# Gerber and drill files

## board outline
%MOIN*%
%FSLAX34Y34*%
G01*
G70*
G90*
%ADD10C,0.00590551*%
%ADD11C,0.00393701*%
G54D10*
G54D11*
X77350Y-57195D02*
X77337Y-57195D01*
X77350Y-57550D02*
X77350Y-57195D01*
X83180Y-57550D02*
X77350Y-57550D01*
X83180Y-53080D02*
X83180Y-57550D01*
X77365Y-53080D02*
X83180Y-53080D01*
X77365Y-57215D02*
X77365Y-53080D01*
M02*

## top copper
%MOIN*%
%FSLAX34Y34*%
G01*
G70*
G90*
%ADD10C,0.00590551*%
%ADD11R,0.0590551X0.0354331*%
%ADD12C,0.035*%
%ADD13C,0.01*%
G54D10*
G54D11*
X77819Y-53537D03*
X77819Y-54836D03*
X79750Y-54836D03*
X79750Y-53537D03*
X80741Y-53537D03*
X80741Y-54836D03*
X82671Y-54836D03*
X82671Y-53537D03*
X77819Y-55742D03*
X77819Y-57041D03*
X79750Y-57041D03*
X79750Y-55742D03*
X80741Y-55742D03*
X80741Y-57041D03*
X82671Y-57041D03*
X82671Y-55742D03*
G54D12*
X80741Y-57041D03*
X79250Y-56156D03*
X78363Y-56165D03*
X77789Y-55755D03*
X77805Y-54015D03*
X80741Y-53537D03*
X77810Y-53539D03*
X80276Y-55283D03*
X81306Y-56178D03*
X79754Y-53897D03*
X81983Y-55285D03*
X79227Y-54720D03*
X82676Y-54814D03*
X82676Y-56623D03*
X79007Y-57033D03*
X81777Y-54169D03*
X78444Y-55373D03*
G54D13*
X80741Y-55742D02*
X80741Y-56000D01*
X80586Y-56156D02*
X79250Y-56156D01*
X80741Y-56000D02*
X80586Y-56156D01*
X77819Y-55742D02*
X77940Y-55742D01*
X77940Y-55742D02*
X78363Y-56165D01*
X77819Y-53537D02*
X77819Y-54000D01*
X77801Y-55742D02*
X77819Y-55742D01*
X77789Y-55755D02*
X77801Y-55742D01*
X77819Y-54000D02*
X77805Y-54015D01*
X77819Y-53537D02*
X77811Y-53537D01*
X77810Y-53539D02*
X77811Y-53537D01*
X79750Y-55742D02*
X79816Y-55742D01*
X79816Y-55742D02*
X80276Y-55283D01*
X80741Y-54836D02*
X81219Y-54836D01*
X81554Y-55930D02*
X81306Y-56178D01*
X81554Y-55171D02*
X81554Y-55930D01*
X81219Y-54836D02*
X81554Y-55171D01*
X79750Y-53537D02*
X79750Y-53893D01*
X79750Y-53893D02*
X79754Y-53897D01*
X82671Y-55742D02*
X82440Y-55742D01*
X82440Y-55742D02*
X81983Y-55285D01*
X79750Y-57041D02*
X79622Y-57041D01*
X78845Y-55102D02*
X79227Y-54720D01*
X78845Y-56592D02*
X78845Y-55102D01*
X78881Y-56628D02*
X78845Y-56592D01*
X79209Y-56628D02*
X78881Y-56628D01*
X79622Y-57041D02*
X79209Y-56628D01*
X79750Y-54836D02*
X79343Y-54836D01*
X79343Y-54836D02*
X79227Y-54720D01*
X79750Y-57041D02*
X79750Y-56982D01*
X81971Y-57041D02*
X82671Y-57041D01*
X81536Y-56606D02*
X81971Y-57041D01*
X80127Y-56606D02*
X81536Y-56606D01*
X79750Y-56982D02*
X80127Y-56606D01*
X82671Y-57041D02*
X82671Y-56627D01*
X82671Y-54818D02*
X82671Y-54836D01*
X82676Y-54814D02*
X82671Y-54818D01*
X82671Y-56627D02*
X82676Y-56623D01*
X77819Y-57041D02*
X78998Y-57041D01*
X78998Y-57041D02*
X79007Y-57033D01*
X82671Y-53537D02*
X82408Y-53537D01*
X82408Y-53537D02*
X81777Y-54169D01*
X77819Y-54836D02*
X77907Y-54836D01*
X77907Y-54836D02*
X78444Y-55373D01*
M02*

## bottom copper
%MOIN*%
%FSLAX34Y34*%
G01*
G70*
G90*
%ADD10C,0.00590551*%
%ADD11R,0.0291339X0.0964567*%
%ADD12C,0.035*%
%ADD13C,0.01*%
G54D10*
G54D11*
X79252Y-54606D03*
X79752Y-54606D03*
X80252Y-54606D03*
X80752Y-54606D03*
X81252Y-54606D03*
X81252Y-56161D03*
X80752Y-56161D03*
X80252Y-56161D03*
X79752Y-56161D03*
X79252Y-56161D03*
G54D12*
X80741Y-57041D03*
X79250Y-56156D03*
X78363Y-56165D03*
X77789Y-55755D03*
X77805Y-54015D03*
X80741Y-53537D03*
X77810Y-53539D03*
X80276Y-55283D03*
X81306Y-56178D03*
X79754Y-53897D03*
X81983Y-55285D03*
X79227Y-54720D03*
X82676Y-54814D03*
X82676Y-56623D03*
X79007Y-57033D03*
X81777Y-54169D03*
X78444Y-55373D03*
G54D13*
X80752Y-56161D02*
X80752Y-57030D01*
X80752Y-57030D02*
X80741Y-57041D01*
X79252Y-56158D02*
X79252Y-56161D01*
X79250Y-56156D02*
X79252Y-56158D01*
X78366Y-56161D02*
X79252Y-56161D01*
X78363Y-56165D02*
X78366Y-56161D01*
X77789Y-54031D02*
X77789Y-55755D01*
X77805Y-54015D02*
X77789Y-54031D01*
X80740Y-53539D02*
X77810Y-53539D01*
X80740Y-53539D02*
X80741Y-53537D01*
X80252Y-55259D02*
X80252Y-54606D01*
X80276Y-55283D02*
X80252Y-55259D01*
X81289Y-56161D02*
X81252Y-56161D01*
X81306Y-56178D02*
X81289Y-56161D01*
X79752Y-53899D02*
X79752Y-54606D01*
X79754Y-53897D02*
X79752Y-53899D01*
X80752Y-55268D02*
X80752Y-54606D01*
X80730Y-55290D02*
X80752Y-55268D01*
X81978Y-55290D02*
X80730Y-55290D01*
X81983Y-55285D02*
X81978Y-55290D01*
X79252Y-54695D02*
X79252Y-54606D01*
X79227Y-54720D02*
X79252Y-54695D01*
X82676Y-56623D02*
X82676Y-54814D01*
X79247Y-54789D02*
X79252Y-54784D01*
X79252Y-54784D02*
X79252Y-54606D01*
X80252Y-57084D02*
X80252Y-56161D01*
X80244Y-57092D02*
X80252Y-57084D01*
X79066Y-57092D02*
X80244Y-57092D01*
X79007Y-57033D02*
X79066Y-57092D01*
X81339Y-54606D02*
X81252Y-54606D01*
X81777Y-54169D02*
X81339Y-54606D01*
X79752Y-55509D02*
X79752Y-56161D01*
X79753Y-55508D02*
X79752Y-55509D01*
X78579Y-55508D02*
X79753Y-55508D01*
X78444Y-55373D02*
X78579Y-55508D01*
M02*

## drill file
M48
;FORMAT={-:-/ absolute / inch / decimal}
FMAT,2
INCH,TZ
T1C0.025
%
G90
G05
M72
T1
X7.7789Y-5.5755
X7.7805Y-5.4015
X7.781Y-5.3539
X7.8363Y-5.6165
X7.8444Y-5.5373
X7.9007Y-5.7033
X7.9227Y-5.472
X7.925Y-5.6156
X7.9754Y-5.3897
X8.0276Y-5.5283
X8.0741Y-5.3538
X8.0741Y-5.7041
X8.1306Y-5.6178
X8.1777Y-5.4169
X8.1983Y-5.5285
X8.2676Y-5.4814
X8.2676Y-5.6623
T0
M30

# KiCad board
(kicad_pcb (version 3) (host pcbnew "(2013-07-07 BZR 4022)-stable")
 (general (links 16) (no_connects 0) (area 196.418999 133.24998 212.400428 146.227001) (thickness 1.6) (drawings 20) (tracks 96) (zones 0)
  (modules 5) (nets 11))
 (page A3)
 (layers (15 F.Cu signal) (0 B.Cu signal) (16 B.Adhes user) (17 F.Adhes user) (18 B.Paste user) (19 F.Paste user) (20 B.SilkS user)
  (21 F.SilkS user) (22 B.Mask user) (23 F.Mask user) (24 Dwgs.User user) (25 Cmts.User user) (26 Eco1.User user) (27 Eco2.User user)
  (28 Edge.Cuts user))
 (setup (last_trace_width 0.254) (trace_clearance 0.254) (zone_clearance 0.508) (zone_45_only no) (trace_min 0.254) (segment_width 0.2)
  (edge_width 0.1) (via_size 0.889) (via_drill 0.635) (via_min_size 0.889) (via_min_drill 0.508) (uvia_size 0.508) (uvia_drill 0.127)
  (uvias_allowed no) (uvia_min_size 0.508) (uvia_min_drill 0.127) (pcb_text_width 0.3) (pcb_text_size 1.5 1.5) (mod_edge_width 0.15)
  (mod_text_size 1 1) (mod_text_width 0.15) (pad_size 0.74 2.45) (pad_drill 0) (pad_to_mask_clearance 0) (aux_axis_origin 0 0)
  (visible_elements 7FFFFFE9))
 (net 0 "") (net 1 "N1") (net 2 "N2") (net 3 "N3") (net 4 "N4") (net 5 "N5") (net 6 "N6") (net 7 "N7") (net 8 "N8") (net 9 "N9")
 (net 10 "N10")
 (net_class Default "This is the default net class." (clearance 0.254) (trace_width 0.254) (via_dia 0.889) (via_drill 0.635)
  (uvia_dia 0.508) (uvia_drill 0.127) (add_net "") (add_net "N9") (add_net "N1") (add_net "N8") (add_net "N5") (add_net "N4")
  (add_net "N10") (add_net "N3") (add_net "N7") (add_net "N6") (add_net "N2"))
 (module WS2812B (layer F.Cu) (at 200.1139 137.63498)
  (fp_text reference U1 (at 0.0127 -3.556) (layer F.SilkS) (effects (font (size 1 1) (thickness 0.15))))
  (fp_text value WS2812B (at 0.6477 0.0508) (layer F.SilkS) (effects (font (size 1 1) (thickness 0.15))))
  (pad 1 smd rect (at -2.45184 -1.64878) (size 1.5 0.9) (layers F.Cu F.Paste F.Mask) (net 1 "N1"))
  (pad 2 smd rect (at -2.45184 1.64878) (size 1.5 0.9) (layers F.Cu F.Paste F.Mask) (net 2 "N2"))
  (pad 3 smd rect (at 2.45184 1.64878) (size 1.5 0.9) (layers F.Cu F.Paste F.Mask) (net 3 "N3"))
  (pad 4 smd rect (at 2.45184 -1.64878) (size 1.5 0.9) (layers F.Cu F.Paste F.Mask) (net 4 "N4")))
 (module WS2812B (layer F.Cu) (at 207.53484 137.63498)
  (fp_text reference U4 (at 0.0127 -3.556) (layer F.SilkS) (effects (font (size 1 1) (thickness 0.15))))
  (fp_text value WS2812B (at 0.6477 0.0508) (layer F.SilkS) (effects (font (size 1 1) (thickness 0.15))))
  (pad 1 smd rect (at -2.45184 -1.64878) (size 1.5 0.9) (layers F.Cu F.Paste F.Mask) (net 1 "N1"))
  (pad 2 smd rect (at -2.45184 1.64878) (size 1.5 0.9) (layers F.Cu F.Paste F.Mask) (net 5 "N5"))
  (pad 3 smd rect (at 2.45184 1.64878) (size 1.5 0.9) (layers F.Cu F.Paste F.Mask) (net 3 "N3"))
  (pad 4 smd rect (at 2.45184 -1.64878) (size 1.5 0.9) (layers F.Cu F.Paste F.Mask) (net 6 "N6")))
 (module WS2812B (layer F.Cu) (at 200.1139 143.23568)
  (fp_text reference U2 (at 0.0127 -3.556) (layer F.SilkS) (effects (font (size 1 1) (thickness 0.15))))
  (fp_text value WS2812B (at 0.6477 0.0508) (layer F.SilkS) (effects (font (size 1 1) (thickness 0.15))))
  (pad 1 smd rect (at -2.45184 -1.64878) (size 1.5 0.9) (layers F.Cu F.Paste F.Mask) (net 1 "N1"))
  (pad 2 smd rect (at -2.45184 1.64878) (size 1.5 0.9) (layers F.Cu F.Paste F.Mask) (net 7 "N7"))
  (pad 3 smd rect (at 2.45184 1.64878) (size 1.5 0.9) (layers F.Cu F.Paste F.Mask) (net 3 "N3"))
  (pad 4 smd rect (at 2.45184 -1.64878) (size 1.5 0.9) (layers F.Cu F.Paste F.Mask) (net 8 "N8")))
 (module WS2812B (layer F.Cu) (at 207.53484 143.23568)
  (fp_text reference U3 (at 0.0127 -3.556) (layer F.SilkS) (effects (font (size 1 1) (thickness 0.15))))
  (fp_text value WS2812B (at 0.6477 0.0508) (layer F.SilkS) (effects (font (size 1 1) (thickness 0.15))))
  (pad 1 smd rect (at -2.45184 -1.64878) (size 1.5 0.9) (layers F.Cu F.Paste F.Mask) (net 1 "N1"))
  (pad 2 smd rect (at -2.45184 1.64878) (size 1.5 0.9) (layers F.Cu F.Paste F.Mask) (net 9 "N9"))
  (pad 3 smd rect (at 2.45184 1.64878) (size 1.5 0.9) (layers F.Cu F.Paste F.Mask) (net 3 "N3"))
  (pad 4 smd rect (at 2.45184 -1.64878) (size 1.5 0.9) (layers F.Cu F.Paste F.Mask) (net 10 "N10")))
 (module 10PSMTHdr (layer F.Cu) (at 207.01 139.7)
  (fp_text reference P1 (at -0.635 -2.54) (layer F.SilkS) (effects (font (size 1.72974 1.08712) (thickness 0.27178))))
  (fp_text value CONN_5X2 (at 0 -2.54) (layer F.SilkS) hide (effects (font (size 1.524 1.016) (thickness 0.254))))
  (pad 2 smd rect (at -5.70992 -1) (size 0.74 2.45) (layers B.Cu B.Paste B.Mask) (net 3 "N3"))
  (pad 4 smd rect (at -4.43992 -1) (size 0.74 2.45) (layers B.Cu B.Paste B.Mask) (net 4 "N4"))
  (pad 6 smd rect (at -3.16992 -1) (size 0.74 2.45) (layers B.Cu B.Paste B.Mask) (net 8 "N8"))
  (pad 8 smd rect (at -1.89992 -1) (size 0.74 2.45) (layers B.Cu B.Paste B.Mask) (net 10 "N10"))
  (pad 10 smd rect (at -0.62992 -1) (size 0.74 2.45) (layers B.Cu B.Paste B.Mask) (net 6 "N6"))
  (pad 9 smd rect (at -0.62992 2.95) (size 0.74 2.45) (layers B.Cu B.Paste B.Mask) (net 5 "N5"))
  (pad 7 smd rect (at -1.89992 2.95) (size 0.74 2.45) (layers B.Cu B.Paste B.Mask) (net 9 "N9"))
  (pad 5 smd rect (at -3.16992 2.95) (size 0.74 2.45) (layers B.Cu B.Paste B.Mask) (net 7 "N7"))
  (pad 3 smd rect (at -4.43992 2.95) (size 0.74 2.45) (layers B.Cu B.Paste B.Mask) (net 2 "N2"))
  (pad 1 smd rect (at -5.70992 2.95) (size 0.74 2.45) (layers B.Cu B.Paste B.Mask) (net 1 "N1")))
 (gr_line (start 196.469 145.2753) (end 196.43598 145.2753) (angle 90) (layer Edge.Cuts) (width 0.1))
 (gr_line (start 196.469 146.177) (end 196.469 145.2753) (angle 90) (layer Edge.Cuts) (width 0.1))
 (gr_line (start 211.2772 146.177) (end 196.469 146.177) (angle 90) (layer Edge.Cuts) (width 0.1))
 (gr_line (start 211.2772 134.8232) (end 211.2772 146.177) (angle 90) (layer Edge.Cuts) (width 0.1))
 (gr_line (start 196.5071 134.8232) (end 211.2772 134.8232) (angle 90) (layer Edge.Cuts) (width 0.1))
 (gr_line (start 196.5071 145.3261) (end 196.5071 134.8232) (angle 90) (layer Edge.Cuts) (width 0.1))
 (via (at 205.083 144.88446) (size 0.889) (layers F.Cu B.Cu) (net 9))
 (segment (start 205.11008 142.65) (end 205.11008 144.85738) (width 0.254) (layer B.Cu) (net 9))
 (segment (start 205.11008 144.85738) (end 205.083 144.88446) (width 0.254) (layer B.Cu) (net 9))
 (segment (start 205.083 141.5869) (end 205.083 142.24168) (width 0.254) (layer F.Cu) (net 1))
 (segment (start 201.30008 142.64132) (end 201.30008 142.65) (width 0.254) (layer B.Cu) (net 1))
 (segment (start 201.295 142.63624) (end 201.30008 142.64132) (width 0.254) (layer B.Cu) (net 1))
 (via (at 201.295 142.63624) (size 0.889) (layers F.Cu B.Cu) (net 1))
 (segment (start 204.68844 142.63624) (end 201.295 142.63624) (width 0.254) (layer F.Cu) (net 1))
 (segment (start 205.083 142.24168) (end 204.68844 142.63624) (width 0.254) (layer F.Cu) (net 1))
 (segment (start 197.66206 141.5869) (end 197.96982 141.5869) (width 0.254) (layer F.Cu) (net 1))
 (segment (start 199.05112 142.65) (end 201.30008 142.65) (width 0.254) (layer B.Cu) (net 1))
 (segment (start 199.04202 142.6591) (end 199.05112 142.65) (width 0.254) (layer B.Cu) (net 1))
 (via (at 199.04202 142.6591) (size 0.889) (layers F.Cu B.Cu) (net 1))
 (segment (start 197.96982 141.5869) (end 199.04202 142.6591) (width 0.254) (layer F.Cu) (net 1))
 (segment (start 197.66206 135.9862) (end 197.66206 137.16074) (width 0.254) (layer F.Cu) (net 1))
 (segment (start 197.61486 141.5869) (end 197.66206 141.5869) (width 0.254) (layer F.Cu) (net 1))
 (segment (start 197.58406 141.6177) (end 197.61486 141.5869) (width 0.254) (layer F.Cu) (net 1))
 (via (at 197.58406 141.6177) (size 0.889) (layers F.Cu B.Cu) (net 1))
 (segment (start 197.58406 137.23874) (end 197.58406 141.6177) (width 0.254) (layer B.Cu) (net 1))
 (segment (start 197.6247 137.1981) (end 197.58406 137.23874) (width 0.254) (layer B.Cu) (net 1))
 (via (at 197.6247 137.1981) (size 0.889) (layers F.Cu B.Cu) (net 1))
 (segment (start 197.66206 137.16074) (end 197.6247 137.1981) (width 0.254) (layer F.Cu) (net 1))
 (via (at 205.083 135.9862) (size 0.889) (layers F.Cu B.Cu) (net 1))
 (segment (start 197.66206 135.9862) (end 197.64026 135.9862) (width 0.254) (layer F.Cu) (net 1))
 (segment (start 197.6374 135.98906) (end 197.64026 135.9862) (width 0.254) (layer F.Cu) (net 1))
 (via (at 197.6374 135.98906) (size 0.889) (layers F.Cu B.Cu) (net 1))
 (segment (start 205.08014 135.98906) (end 197.6374 135.98906) (width 0.254) (layer B.Cu) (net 1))
 (segment (start 205.08014 135.98906) (end 205.083 135.9862) (width 0.254) (layer B.Cu) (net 1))
 (segment (start 202.56574 141.5869) (end 202.73296 141.5869) (width 0.254) (layer F.Cu) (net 8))
 (segment (start 203.84008 140.35786) (end 203.84008 138.7) (width 0.254) (layer B.Cu) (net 8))
 (segment (start 203.90104 140.41882) (end 203.84008 140.35786) (width 0.254) (layer B.Cu) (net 8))
 (via (at 203.90104 140.41882) (size 0.889) (layers F.Cu B.Cu) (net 8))
 (segment (start 202.73296 141.5869) (end 203.90104 140.41882) (width 0.254) (layer F.Cu) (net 8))
 (segment (start 205.083 139.28376) (end 206.29658 139.28376) (width 0.254) (layer F.Cu) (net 5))
 (segment (start 206.47512 142.65) (end 206.38008 142.65) (width 0.254) (layer B.Cu) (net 5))
 (segment (start 206.51724 142.69212) (end 206.47512 142.65) (width 0.254) (layer B.Cu) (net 5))
 (via (at 206.51724 142.69212) (size 0.889) (layers F.Cu B.Cu) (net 5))
 (segment (start 207.14716 142.0622) (end 206.51724 142.69212) (width 0.254) (layer F.Cu) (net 5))
 (segment (start 207.14716 140.13434) (end 207.14716 142.0622) (width 0.254) (layer F.Cu) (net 5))
 (segment (start 206.29658 139.28376) (end 207.14716 140.13434) (width 0.254) (layer F.Cu) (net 5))
 (segment (start 202.56574 135.9862) (end 202.56574 136.88896) (width 0.254) (layer F.Cu) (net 4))
 (segment (start 202.57008 136.90346) (end 202.57008 138.7) (width 0.254) (layer B.Cu) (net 4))
 (segment (start 202.57516 136.89838) (end 202.57008 136.90346) (width 0.254) (layer B.Cu) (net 4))
 (via (at 202.57516 136.89838) (size 0.889) (layers F.Cu B.Cu) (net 4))
 (segment (start 202.56574 136.88896) (end 202.57516 136.89838) (width 0.254) (layer F.Cu) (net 4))
 (segment (start 209.98668 141.5869) (end 209.39982 141.5869) (width 0.254) (layer F.Cu) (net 10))
 (segment (start 205.11008 140.38072) (end 205.11008 138.7) (width 0.254) (layer B.Cu) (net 10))
 (segment (start 205.0542 140.4366) (end 205.11008 140.38072) (width 0.254) (layer B.Cu) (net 10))
 (segment (start 208.22412 140.4366) (end 205.0542 140.4366) (width 0.254) (layer B.Cu) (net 10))
 (segment (start 208.23682 140.4239) (end 208.22412 140.4366) (width 0.254) (layer B.Cu) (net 10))
 (via (at 208.23682 140.4239) (size 0.889) (layers F.Cu B.Cu) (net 10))
 (segment (start 209.39982 141.5869) (end 208.23682 140.4239) (width 0.254) (layer F.Cu) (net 10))
 (segment (start 202.56574 144.88446) (end 202.2402 144.88446) (width 0.254) (layer F.Cu) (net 3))
 (segment (start 200.2663 139.95908) (end 201.23658 138.9888) (width 0.254) (layer F.Cu) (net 3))
 (segment (start 200.2663 143.74368) (end 200.2663 139.95908) (width 0.254) (layer F.Cu) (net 3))
 (segment (start 200.35774 143.83512) (end 200.2663 143.74368) (width 0.254) (layer F.Cu) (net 3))
 (segment (start 201.19086 143.83512) (end 200.35774 143.83512) (width 0.254) (layer F.Cu) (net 3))
 (segment (start 202.2402 144.88446) (end 201.19086 143.83512) (width 0.254) (layer F.Cu) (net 3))
 (segment (start 202.56574 139.28376) (end 201.53154 139.28376) (width 0.254) (layer F.Cu) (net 3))
 (segment (start 201.53154 139.28376) (end 201.23658 138.9888) (width 0.254) (layer F.Cu) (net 3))
 (segment (start 201.30008 138.9253) (end 201.30008 138.7) (width 0.254) (layer B.Cu) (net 3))
 (via (at 201.23658 138.9888) (size 0.889) (layers F.Cu B.Cu) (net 3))
 (segment (start 201.23658 138.9888) (end 201.30008 138.9253) (width 0.254) (layer B.Cu) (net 3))
 (segment (start 202.56574 144.88446) (end 202.56574 144.73608) (width 0.254) (layer F.Cu) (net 3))
 (segment (start 208.20666 144.88446) (end 209.98668 144.88446) (width 0.254) (layer F.Cu) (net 3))
 (segment (start 207.10144 143.77924) (end 208.20666 144.88446) (width 0.254) (layer F.Cu) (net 3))
 (segment (start 203.52258 143.77924) (end 207.10144 143.77924) (width 0.254) (layer F.Cu) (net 3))
 (segment (start 202.56574 144.73608) (end 203.52258 143.77924) (width 0.254) (layer F.Cu) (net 3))
 (segment (start 209.98668 144.88446) (end 209.98668 143.83278) (width 0.254) (layer F.Cu) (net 3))
 (segment (start 209.98668 139.23792) (end 209.98668 139.28376) (width 0.254) (layer F.Cu) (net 3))
 (segment (start 209.99704 139.22756) (end 209.98668 139.23792) (width 0.254) (layer F.Cu) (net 3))
 (via (at 209.99704 139.22756) (size 0.889) (layers F.Cu B.Cu) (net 3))
 (segment (start 209.99704 143.82242) (end 209.99704 139.22756) (width 0.254) (layer B.Cu) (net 3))
 (via (at 209.99704 143.82242) (size 0.889) (layers F.Cu B.Cu) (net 3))
 (segment (start 209.98668 143.83278) (end 209.99704 143.82242) (width 0.254) (layer F.Cu) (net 3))
 (segment (start 201.28738 139.16406) (end 201.30008 139.15136) (width 0.254) (layer B.Cu) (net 3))
 (segment (start 201.30008 139.15136) (end 201.30008 138.7) (width 0.254) (layer B.Cu) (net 3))
 (segment (start 197.66206 144.88446) (end 200.65714 144.88446) (width 0.254) (layer F.Cu) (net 7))
 (segment (start 203.84008 144.99336) (end 203.84008 142.65) (width 0.254) (layer B.Cu) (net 7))
 (segment (start 203.81976 145.01368) (end 203.84008 144.99336) (width 0.254) (layer B.Cu) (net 7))
 (segment (start 200.82764 145.01368) (end 203.81976 145.01368) (width 0.254) (layer B.Cu) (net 7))
 (segment (start 200.67778 144.86382) (end 200.82764 145.01368) (width 0.254) (layer B.Cu) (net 7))
 (via (at 200.67778 144.86382) (size 0.889) (layers F.Cu B.Cu) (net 7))
 (segment (start 200.65714 144.88446) (end 200.67778 144.86382) (width 0.254) (layer F.Cu) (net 7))
 (segment (start 209.98668 135.9862) (end 209.31664 135.9862) (width 0.254) (layer F.Cu) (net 6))
 (segment (start 206.60284 138.7) (end 206.38008 138.7) (width 0.254) (layer B.Cu) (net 6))
 (segment (start 207.71358 137.58926) (end 206.60284 138.7) (width 0.254) (layer B.Cu) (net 6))
 (via (at 207.71358 137.58926) (size 0.889) (layers F.Cu B.Cu) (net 6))
 (segment (start 209.31664 135.9862) (end 207.71358 137.58926) (width 0.254) (layer F.Cu) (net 6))
 (segment (start 197.66206 139.28376) (end 197.8841 139.28376) (width 0.254) (layer F.Cu) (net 2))
 (segment (start 202.57008 140.99286) (end 202.57008 142.65) (width 0.254) (layer B.Cu) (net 2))
 (segment (start 202.57262 140.99032) (end 202.57008 140.99286) (width 0.254) (layer B.Cu) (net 2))
 (segment (start 199.59066 140.99032) (end 202.57262 140.99032) (width 0.254) (layer B.Cu) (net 2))
 (segment (start 199.24776 140.64742) (end 199.59066 140.99032) (width 0.254) (layer B.Cu) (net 2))
 (via (at 199.24776 140.64742) (size 0.889) (layers F.Cu B.Cu) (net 2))
 (segment (start 197.8841 139.28376) (end 199.24776 140.64742) (width 0.254) (layer F.Cu) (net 2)))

